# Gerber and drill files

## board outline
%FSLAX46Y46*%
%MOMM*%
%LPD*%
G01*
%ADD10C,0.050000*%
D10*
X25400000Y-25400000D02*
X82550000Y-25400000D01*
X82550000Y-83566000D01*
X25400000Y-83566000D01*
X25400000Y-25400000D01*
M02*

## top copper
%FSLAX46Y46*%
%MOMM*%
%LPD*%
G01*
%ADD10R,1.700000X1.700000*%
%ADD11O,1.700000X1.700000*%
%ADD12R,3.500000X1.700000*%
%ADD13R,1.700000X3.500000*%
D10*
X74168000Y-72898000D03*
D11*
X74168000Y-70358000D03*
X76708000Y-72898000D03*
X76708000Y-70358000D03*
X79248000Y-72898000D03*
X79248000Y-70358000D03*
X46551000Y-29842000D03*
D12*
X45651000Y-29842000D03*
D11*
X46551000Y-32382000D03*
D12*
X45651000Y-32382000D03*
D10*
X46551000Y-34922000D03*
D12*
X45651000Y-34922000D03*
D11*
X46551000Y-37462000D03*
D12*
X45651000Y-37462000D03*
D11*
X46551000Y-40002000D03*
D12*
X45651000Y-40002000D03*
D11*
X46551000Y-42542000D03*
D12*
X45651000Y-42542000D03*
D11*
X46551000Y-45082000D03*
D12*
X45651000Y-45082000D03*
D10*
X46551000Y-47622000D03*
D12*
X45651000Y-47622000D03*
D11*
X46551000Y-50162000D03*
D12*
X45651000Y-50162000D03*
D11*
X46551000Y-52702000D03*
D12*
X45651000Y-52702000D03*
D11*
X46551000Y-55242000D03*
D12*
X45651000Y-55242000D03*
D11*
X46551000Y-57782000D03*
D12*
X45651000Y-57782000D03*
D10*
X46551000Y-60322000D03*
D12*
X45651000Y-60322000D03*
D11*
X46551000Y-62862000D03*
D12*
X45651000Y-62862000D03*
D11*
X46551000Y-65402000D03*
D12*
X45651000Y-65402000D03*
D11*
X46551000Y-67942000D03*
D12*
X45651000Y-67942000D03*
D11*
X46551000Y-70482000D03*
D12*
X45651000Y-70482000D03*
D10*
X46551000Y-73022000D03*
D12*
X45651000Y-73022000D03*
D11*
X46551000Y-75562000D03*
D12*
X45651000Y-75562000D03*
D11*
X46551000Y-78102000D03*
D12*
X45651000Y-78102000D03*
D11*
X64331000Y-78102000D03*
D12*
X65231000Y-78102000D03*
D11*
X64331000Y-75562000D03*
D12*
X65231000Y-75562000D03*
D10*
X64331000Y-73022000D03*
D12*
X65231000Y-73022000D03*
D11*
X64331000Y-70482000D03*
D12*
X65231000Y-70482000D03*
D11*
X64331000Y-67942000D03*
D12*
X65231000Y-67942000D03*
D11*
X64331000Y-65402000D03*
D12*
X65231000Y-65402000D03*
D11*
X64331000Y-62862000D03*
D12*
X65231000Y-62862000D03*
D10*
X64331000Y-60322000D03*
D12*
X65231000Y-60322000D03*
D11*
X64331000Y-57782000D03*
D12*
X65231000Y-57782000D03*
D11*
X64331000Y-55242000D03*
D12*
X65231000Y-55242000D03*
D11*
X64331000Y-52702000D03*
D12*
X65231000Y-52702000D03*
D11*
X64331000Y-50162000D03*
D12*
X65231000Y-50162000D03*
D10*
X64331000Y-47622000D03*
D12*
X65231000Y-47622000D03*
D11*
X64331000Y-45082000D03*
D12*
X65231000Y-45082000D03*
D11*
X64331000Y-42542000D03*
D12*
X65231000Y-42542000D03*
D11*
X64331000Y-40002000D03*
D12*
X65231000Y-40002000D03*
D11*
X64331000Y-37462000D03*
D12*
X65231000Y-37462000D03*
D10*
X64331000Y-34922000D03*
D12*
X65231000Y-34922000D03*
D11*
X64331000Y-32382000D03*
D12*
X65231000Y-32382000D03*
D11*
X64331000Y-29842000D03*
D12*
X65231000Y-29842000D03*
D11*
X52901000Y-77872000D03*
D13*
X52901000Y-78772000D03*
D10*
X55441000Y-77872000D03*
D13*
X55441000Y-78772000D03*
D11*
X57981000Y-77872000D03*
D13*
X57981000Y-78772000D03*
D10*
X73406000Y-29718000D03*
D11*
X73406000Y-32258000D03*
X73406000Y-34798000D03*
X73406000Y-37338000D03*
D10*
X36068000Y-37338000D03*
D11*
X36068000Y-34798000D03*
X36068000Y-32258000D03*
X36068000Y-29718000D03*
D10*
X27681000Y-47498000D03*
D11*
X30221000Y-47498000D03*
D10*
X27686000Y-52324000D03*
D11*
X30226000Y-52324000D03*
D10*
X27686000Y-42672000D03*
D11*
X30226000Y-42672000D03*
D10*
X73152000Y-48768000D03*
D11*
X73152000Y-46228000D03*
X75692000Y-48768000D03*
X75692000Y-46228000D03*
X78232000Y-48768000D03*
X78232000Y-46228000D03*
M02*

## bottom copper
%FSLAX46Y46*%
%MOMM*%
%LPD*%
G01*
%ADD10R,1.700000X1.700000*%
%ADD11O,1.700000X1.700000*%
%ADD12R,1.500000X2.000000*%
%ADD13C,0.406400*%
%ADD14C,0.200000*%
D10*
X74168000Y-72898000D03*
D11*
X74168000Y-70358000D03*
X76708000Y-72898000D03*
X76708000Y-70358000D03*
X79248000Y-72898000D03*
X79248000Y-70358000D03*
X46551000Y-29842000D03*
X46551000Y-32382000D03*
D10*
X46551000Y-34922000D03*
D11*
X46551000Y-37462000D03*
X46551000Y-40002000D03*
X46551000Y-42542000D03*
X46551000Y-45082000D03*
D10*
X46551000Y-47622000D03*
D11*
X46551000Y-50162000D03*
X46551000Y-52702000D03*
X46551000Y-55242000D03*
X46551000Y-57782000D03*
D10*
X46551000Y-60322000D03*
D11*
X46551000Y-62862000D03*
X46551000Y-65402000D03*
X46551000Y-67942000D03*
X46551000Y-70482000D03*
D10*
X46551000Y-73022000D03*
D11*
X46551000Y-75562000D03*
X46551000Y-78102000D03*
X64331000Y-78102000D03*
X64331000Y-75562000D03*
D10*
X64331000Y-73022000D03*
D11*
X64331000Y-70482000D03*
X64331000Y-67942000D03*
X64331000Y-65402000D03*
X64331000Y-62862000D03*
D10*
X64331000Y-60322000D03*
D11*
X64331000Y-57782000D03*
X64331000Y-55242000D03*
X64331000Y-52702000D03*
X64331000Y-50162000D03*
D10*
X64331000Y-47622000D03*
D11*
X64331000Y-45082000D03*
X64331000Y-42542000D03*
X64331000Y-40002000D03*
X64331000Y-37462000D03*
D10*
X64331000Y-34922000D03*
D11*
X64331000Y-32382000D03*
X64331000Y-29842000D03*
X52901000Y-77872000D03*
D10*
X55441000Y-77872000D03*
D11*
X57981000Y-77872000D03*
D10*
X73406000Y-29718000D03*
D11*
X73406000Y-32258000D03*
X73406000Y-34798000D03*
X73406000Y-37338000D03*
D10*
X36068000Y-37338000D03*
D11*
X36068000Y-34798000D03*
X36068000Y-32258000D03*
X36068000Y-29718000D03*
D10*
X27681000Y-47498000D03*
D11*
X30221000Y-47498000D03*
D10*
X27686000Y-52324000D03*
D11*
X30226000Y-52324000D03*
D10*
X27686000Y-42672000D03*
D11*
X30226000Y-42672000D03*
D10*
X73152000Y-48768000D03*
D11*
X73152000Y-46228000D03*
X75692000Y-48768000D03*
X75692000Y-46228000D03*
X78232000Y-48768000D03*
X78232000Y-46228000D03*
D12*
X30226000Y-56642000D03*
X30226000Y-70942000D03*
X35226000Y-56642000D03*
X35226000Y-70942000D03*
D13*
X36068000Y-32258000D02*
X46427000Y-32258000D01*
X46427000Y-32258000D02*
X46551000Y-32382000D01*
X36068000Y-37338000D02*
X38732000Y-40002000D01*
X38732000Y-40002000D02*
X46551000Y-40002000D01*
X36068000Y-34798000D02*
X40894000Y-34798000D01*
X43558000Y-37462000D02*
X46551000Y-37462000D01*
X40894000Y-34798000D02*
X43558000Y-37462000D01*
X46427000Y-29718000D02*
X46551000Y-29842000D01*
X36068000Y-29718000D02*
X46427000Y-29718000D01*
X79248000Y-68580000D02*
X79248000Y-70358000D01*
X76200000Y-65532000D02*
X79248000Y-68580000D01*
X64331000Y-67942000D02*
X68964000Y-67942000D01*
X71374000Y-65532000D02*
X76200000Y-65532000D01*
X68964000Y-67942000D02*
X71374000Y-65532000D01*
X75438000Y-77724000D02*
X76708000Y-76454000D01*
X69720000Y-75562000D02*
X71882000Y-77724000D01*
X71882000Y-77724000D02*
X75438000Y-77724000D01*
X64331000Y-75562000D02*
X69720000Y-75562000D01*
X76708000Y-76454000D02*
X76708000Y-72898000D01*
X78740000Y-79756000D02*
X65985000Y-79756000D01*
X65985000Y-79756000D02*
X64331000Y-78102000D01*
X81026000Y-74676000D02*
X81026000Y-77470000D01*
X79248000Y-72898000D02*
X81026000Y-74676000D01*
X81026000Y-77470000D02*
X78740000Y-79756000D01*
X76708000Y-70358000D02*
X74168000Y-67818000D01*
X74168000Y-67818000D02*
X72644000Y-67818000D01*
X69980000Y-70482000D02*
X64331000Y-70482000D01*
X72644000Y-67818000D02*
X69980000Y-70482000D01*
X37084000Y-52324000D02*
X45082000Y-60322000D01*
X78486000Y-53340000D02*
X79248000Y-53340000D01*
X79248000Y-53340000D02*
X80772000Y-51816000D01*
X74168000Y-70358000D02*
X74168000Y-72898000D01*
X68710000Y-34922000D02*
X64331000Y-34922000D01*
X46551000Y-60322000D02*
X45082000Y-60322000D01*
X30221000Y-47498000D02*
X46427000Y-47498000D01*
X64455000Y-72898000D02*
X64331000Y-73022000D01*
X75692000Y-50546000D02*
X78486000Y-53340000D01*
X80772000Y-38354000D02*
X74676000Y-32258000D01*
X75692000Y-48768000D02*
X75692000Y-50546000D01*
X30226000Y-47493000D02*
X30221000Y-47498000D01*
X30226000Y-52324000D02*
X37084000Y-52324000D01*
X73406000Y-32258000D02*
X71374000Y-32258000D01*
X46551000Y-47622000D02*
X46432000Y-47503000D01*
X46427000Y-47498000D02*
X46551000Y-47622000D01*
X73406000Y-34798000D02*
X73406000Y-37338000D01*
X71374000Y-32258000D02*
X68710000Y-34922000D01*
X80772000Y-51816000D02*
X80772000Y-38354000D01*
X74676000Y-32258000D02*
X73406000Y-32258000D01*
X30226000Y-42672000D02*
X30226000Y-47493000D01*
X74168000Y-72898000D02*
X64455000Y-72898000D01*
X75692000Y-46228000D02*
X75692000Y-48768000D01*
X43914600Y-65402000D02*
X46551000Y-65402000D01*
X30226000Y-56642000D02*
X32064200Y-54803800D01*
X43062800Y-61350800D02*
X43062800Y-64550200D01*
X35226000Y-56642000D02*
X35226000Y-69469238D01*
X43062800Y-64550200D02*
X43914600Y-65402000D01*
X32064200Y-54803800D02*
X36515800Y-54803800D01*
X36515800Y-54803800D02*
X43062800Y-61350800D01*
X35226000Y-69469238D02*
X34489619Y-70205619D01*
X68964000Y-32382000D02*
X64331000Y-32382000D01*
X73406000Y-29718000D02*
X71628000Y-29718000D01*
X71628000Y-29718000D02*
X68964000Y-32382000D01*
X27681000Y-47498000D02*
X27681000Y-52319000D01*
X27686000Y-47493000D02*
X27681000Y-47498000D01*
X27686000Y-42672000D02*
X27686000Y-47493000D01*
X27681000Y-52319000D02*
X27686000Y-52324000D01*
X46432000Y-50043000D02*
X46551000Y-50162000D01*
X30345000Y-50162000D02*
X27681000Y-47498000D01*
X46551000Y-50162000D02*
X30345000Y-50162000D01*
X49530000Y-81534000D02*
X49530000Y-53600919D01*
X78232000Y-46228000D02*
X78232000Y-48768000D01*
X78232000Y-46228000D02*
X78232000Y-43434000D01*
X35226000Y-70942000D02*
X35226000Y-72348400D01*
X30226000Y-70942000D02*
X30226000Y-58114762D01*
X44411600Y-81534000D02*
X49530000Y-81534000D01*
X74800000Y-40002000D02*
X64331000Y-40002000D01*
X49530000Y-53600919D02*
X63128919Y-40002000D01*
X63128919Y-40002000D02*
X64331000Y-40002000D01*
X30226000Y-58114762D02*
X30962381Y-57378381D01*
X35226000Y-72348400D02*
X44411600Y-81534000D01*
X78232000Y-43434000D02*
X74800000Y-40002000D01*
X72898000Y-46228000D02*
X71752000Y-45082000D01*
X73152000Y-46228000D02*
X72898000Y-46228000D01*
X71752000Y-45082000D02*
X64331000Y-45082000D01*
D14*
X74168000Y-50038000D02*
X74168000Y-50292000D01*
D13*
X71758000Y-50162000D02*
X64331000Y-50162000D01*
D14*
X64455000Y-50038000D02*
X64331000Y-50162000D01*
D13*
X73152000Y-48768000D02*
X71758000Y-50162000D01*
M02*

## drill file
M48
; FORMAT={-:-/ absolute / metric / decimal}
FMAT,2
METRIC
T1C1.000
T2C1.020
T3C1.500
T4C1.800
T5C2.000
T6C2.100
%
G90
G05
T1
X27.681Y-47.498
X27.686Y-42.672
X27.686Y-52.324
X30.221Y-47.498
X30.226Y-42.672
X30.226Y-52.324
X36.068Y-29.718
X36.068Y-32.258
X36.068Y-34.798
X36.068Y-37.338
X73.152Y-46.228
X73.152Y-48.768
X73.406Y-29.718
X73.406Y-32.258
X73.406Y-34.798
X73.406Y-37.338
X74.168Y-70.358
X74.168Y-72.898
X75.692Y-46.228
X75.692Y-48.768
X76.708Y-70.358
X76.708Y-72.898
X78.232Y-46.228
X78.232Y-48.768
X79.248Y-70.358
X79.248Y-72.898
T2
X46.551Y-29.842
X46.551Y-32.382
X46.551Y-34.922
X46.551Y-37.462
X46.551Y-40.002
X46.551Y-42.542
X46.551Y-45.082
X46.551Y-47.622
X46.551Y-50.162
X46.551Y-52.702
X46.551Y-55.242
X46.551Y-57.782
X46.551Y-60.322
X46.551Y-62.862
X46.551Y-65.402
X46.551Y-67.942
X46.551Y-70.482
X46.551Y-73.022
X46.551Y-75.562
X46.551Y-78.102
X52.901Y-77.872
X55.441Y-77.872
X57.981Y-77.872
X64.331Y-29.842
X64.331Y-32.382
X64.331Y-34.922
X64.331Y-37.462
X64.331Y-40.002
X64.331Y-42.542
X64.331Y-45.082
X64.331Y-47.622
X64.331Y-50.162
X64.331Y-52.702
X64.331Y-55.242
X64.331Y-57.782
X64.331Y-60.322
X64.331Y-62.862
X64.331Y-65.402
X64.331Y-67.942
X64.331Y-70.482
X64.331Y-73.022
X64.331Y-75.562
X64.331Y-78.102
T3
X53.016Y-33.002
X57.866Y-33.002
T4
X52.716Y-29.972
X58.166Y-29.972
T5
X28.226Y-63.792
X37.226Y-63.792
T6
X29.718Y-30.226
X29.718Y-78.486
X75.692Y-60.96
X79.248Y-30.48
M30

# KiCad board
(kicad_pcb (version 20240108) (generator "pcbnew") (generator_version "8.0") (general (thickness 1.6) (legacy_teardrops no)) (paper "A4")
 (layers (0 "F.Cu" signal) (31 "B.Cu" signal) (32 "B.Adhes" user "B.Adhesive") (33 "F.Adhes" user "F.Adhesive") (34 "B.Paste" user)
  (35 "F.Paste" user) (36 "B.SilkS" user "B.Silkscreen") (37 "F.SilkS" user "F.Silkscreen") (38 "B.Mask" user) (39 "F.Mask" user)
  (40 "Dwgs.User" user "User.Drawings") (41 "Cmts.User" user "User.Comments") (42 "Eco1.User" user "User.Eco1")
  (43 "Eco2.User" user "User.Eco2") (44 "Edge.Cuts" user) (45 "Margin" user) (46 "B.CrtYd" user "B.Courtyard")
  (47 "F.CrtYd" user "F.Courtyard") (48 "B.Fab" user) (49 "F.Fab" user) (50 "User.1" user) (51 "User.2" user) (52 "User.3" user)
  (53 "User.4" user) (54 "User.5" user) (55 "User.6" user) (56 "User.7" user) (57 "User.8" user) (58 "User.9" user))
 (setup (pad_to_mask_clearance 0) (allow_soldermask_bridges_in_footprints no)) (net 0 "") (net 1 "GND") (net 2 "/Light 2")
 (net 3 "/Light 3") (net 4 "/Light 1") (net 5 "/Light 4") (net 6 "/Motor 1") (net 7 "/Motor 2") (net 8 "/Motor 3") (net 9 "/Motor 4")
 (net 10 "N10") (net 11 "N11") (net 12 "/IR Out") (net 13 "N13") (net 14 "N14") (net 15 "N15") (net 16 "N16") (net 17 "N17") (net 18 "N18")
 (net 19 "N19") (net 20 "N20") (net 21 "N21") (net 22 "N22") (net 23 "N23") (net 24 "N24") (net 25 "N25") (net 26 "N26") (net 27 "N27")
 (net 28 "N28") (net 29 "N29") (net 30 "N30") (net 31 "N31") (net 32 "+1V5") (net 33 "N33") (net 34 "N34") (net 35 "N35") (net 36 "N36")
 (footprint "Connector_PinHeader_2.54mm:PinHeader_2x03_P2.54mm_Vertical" (layer "F.Cu") (at 74.168 72.898 90)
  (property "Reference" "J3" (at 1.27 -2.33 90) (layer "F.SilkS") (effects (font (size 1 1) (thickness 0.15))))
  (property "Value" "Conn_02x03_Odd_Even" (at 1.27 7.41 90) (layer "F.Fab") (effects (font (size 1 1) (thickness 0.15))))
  (pad "1" thru_hole rect (at 0 0 90) (size 1.7 1.7) (drill 1) (layers "*.Cu" "*.Mask") (remove_unused_layers no) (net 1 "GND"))
  (pad "2" thru_hole oval (at 2.54 0 90) (size 1.7 1.7) (drill 1) (layers "*.Cu" "*.Mask") (remove_unused_layers no) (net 1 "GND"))
  (pad "3" thru_hole oval (at 0 2.54 90) (size 1.7 1.7) (drill 1) (layers "*.Cu" "*.Mask") (remove_unused_layers no) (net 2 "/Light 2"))
  (pad "4" thru_hole oval (at 2.54 2.54 90) (size 1.7 1.7) (drill 1) (layers "*.Cu" "*.Mask") (remove_unused_layers no) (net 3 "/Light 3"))
  (pad "5" thru_hole oval (at 0 5.08 90) (size 1.7 1.7) (drill 1) (layers "*.Cu" "*.Mask") (remove_unused_layers no) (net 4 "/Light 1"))
  (pad "6" thru_hole oval (at 2.54 5.08 90) (size 1.7 1.7) (drill 1) (layers "*.Cu" "*.Mask") (remove_unused_layers no) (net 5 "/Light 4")))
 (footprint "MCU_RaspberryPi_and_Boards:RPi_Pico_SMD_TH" (layer "F.Cu") (at 55.441 53.972)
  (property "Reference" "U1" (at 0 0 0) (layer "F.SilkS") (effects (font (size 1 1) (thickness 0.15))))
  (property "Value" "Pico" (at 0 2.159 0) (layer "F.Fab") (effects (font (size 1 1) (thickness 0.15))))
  (pad "" np_thru_hole oval (at -2.725 -24) (size 1.8 1.8) (drill 1.8) (layers "*.Cu" "*.Mask"))
  (pad "" np_thru_hole oval (at -2.425 -20.97) (size 1.5 1.5) (drill 1.5) (layers "*.Cu" "*.Mask"))
  (pad "" np_thru_hole oval (at 2.425 -20.97) (size 1.5 1.5) (drill 1.5) (layers "*.Cu" "*.Mask"))
  (pad "" np_thru_hole oval (at 2.725 -24) (size 1.8 1.8) (drill 1.8) (layers "*.Cu" "*.Mask"))
  (pad "1" thru_hole oval (at -8.89 -24.13) (size 1.7 1.7) (drill 1.02) (layers "*.Cu" "*.Mask") (remove_unused_layers no)
   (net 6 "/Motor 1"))
  (pad "1" smd rect (at -8.89 -24.13) (size 3.5 1.7) (drill (offset -0.9 0)) (layers "F.Cu" "F.Mask") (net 6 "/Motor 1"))
  (pad "2" thru_hole oval (at -8.89 -21.59) (size 1.7 1.7) (drill 1.02) (layers "*.Cu" "*.Mask") (remove_unused_layers no)
   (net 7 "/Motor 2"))
  (pad "2" smd rect (at -8.89 -21.59) (size 3.5 1.7) (drill (offset -0.9 0)) (layers "F.Cu" "F.Mask") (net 7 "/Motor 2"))
  (pad "3" thru_hole rect (at -8.89 -19.05) (size 1.7 1.7) (drill 1.02) (layers "*.Cu" "*.Mask") (remove_unused_layers no) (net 1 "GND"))
  (pad "3" smd rect (at -8.89 -19.05) (size 3.5 1.7) (drill (offset -0.9 0)) (layers "F.Cu" "F.Mask") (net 1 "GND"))
  (pad "4" thru_hole oval (at -8.89 -16.51) (size 1.7 1.7) (drill 1.02) (layers "*.Cu" "*.Mask") (remove_unused_layers no)
   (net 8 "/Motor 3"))
  (pad "4" smd rect (at -8.89 -16.51) (size 3.5 1.7) (drill (offset -0.9 0)) (layers "F.Cu" "F.Mask") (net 8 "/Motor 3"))
  (pad "5" thru_hole oval (at -8.89 -13.97) (size 1.7 1.7) (drill 1.02) (layers "*.Cu" "*.Mask") (remove_unused_layers no)
   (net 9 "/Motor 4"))
  (pad "5" smd rect (at -8.89 -13.97) (size 3.5 1.7) (drill (offset -0.9 0)) (layers "F.Cu" "F.Mask") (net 9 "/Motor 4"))
  (pad "6" thru_hole oval (at -8.89 -11.43) (size 1.7 1.7) (drill 1.02) (layers "*.Cu" "*.Mask") (remove_unused_layers no) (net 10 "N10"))
  (pad "6" smd rect (at -8.89 -11.43) (size 3.5 1.7) (drill (offset -0.9 0)) (layers "F.Cu" "F.Mask") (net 10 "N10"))
  (pad "7" thru_hole oval (at -8.89 -8.89) (size 1.7 1.7) (drill 1.02) (layers "*.Cu" "*.Mask") (remove_unused_layers no) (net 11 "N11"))
  (pad "7" smd rect (at -8.89 -8.89) (size 3.5 1.7) (drill (offset -0.9 0)) (layers "F.Cu" "F.Mask") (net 11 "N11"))
  (pad "8" thru_hole rect (at -8.89 -6.35) (size 1.7 1.7) (drill 1.02) (layers "*.Cu" "*.Mask") (remove_unused_layers no) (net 1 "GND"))
  (pad "8" smd rect (at -8.89 -6.35) (size 3.5 1.7) (drill (offset -0.9 0)) (layers "F.Cu" "F.Mask") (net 1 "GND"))
  (pad "9" thru_hole oval (at -8.89 -3.81) (size 1.7 1.7) (drill 1.02) (layers "*.Cu" "*.Mask") (remove_unused_layers no) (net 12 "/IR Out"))
  (pad "9" smd rect (at -8.89 -3.81) (size 3.5 1.7) (drill (offset -0.9 0)) (layers "F.Cu" "F.Mask") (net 12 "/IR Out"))
  (pad "10" thru_hole oval (at -8.89 -1.27) (size 1.7 1.7) (drill 1.02) (layers "*.Cu" "*.Mask") (remove_unused_layers no) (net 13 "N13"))
  (pad "10" smd rect (at -8.89 -1.27) (size 3.5 1.7) (drill (offset -0.9 0)) (layers "F.Cu" "F.Mask") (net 13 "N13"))
  (pad "11" thru_hole oval (at -8.89 1.27) (size 1.7 1.7) (drill 1.02) (layers "*.Cu" "*.Mask") (remove_unused_layers no) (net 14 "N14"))
  (pad "11" smd rect (at -8.89 1.27) (size 3.5 1.7) (drill (offset -0.9 0)) (layers "F.Cu" "F.Mask") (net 14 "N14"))
  (pad "12" thru_hole oval (at -8.89 3.81) (size 1.7 1.7) (drill 1.02) (layers "*.Cu" "*.Mask") (remove_unused_layers no) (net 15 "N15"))
  (pad "12" smd rect (at -8.89 3.81) (size 3.5 1.7) (drill (offset -0.9 0)) (layers "F.Cu" "F.Mask") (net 15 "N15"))
  (pad "13" thru_hole rect (at -8.89 6.35) (size 1.7 1.7) (drill 1.02) (layers "*.Cu" "*.Mask") (remove_unused_layers no) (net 1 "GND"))
  (pad "13" smd rect (at -8.89 6.35) (size 3.5 1.7) (drill (offset -0.9 0)) (layers "F.Cu" "F.Mask") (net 1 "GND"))
  (pad "14" thru_hole oval (at -8.89 8.89) (size 1.7 1.7) (drill 1.02) (layers "*.Cu" "*.Mask") (remove_unused_layers no) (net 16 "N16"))
  (pad "14" smd rect (at -8.89 8.89) (size 3.5 1.7) (drill (offset -0.9 0)) (layers "F.Cu" "F.Mask") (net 16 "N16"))
  (pad "15" thru_hole oval (at -8.89 11.43) (size 1.7 1.7) (drill 1.02) (layers "*.Cu" "*.Mask") (remove_unused_layers no) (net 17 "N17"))
  (pad "15" smd rect (at -8.89 11.43) (size 3.5 1.7) (drill (offset -0.9 0)) (layers "F.Cu" "F.Mask") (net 17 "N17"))
  (pad "16" thru_hole oval (at -8.89 13.97) (size 1.7 1.7) (drill 1.02) (layers "*.Cu" "*.Mask") (remove_unused_layers no) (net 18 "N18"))
  (pad "16" smd rect (at -8.89 13.97) (size 3.5 1.7) (drill (offset -0.9 0)) (layers "F.Cu" "F.Mask") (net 18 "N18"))
  (pad "17" thru_hole oval (at -8.89 16.51) (size 1.7 1.7) (drill 1.02) (layers "*.Cu" "*.Mask") (remove_unused_layers no) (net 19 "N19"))
  (pad "17" smd rect (at -8.89 16.51) (size 3.5 1.7) (drill (offset -0.9 0)) (layers "F.Cu" "F.Mask") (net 19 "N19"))
  (pad "18" thru_hole rect (at -8.89 19.05) (size 1.7 1.7) (drill 1.02) (layers "*.Cu" "*.Mask") (remove_unused_layers no) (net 1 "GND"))
  (pad "18" smd rect (at -8.89 19.05) (size 3.5 1.7) (drill (offset -0.9 0)) (layers "F.Cu" "F.Mask") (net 1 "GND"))
  (pad "19" thru_hole oval (at -8.89 21.59) (size 1.7 1.7) (drill 1.02) (layers "*.Cu" "*.Mask") (remove_unused_layers no) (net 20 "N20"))
  (pad "19" smd rect (at -8.89 21.59) (size 3.5 1.7) (drill (offset -0.9 0)) (layers "F.Cu" "F.Mask") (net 20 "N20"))
  (pad "20" thru_hole oval (at -8.89 24.13) (size 1.7 1.7) (drill 1.02) (layers "*.Cu" "*.Mask") (remove_unused_layers no) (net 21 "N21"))
  (pad "20" smd rect (at -8.89 24.13) (size 3.5 1.7) (drill (offset -0.9 0)) (layers "F.Cu" "F.Mask") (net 21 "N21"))
  (pad "21" thru_hole oval (at 8.89 24.13) (size 1.7 1.7) (drill 1.02) (layers "*.Cu" "*.Mask") (remove_unused_layers no) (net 4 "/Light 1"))
  (pad "21" smd rect (at 8.89 24.13) (size 3.5 1.7) (drill (offset 0.9 0)) (layers "F.Cu" "F.Mask") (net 4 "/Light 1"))
  (pad "22" thru_hole oval (at 8.89 21.59) (size 1.7 1.7) (drill 1.02) (layers "*.Cu" "*.Mask") (remove_unused_layers no) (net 2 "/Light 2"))
  (pad "22" smd rect (at 8.89 21.59) (size 3.5 1.7) (drill (offset 0.9 0)) (layers "F.Cu" "F.Mask") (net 2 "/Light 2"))
  (pad "23" thru_hole rect (at 8.89 19.05) (size 1.7 1.7) (drill 1.02) (layers "*.Cu" "*.Mask") (remove_unused_layers no) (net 1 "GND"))
  (pad "23" smd rect (at 8.89 19.05) (size 3.5 1.7) (drill (offset 0.9 0)) (layers "F.Cu" "F.Mask") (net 1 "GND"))
  (pad "24" thru_hole oval (at 8.89 16.51) (size 1.7 1.7) (drill 1.02) (layers "*.Cu" "*.Mask") (remove_unused_layers no) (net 3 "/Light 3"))
  (pad "24" smd rect (at 8.89 16.51) (size 3.5 1.7) (drill (offset 0.9 0)) (layers "F.Cu" "F.Mask") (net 3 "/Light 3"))
  (pad "25" thru_hole oval (at 8.89 13.97) (size 1.7 1.7) (drill 1.02) (layers "*.Cu" "*.Mask") (remove_unused_layers no) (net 5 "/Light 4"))
  (pad "25" smd rect (at 8.89 13.97) (size 3.5 1.7) (drill (offset 0.9 0)) (layers "F.Cu" "F.Mask") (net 5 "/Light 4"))
  (pad "26" thru_hole oval (at 8.89 11.43) (size 1.7 1.7) (drill 1.02) (layers "*.Cu" "*.Mask") (remove_unused_layers no) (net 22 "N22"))
  (pad "26" smd rect (at 8.89 11.43) (size 3.5 1.7) (drill (offset 0.9 0)) (layers "F.Cu" "F.Mask") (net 22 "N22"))
  (pad "27" thru_hole oval (at 8.89 8.89) (size 1.7 1.7) (drill 1.02) (layers "*.Cu" "*.Mask") (remove_unused_layers no) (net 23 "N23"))
  (pad "27" smd rect (at 8.89 8.89) (size 3.5 1.7) (drill (offset 0.9 0)) (layers "F.Cu" "F.Mask") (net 23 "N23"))
  (pad "28" thru_hole rect (at 8.89 6.35) (size 1.7 1.7) (drill 1.02) (layers "*.Cu" "*.Mask") (remove_unused_layers no) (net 1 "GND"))
  (pad "28" smd rect (at 8.89 6.35) (size 3.5 1.7) (drill (offset 0.9 0)) (layers "F.Cu" "F.Mask") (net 1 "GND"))
  (pad "29" thru_hole oval (at 8.89 3.81) (size 1.7 1.7) (drill 1.02) (layers "*.Cu" "*.Mask") (remove_unused_layers no) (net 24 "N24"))
  (pad "29" smd rect (at 8.89 3.81) (size 3.5 1.7) (drill (offset 0.9 0)) (layers "F.Cu" "F.Mask") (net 24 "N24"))
  (pad "30" thru_hole oval (at 8.89 1.27) (size 1.7 1.7) (drill 1.02) (layers "*.Cu" "*.Mask") (remove_unused_layers no) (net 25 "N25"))
  (pad "30" smd rect (at 8.89 1.27) (size 3.5 1.7) (drill (offset 0.9 0)) (layers "F.Cu" "F.Mask") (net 25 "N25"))
  (pad "31" thru_hole oval (at 8.89 -1.27) (size 1.7 1.7) (drill 1.02) (layers "*.Cu" "*.Mask") (remove_unused_layers no) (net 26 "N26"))
  (pad "31" smd rect (at 8.89 -1.27) (size 3.5 1.7) (drill (offset 0.9 0)) (layers "F.Cu" "F.Mask") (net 26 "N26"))
  (pad "32" thru_hole oval (at 8.89 -3.81) (size 1.7 1.7) (drill 1.02) (layers "*.Cu" "*.Mask") (remove_unused_layers no) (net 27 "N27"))
  (pad "32" smd rect (at 8.89 -3.81) (size 3.5 1.7) (drill (offset 0.9 0)) (layers "F.Cu" "F.Mask") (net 27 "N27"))
  (pad "33" thru_hole rect (at 8.89 -6.35) (size 1.7 1.7) (drill 1.02) (layers "*.Cu" "*.Mask") (remove_unused_layers no) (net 1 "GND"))
  (pad "33" smd rect (at 8.89 -6.35) (size 3.5 1.7) (drill (offset 0.9 0)) (layers "F.Cu" "F.Mask") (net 1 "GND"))
  (pad "34" thru_hole oval (at 8.89 -8.89) (size 1.7 1.7) (drill 1.02) (layers "*.Cu" "*.Mask") (remove_unused_layers no) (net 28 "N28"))
  (pad "34" smd rect (at 8.89 -8.89) (size 3.5 1.7) (drill (offset 0.9 0)) (layers "F.Cu" "F.Mask") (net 28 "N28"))
  (pad "35" thru_hole oval (at 8.89 -11.43) (size 1.7 1.7) (drill 1.02) (layers "*.Cu" "*.Mask") (remove_unused_layers no) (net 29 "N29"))
  (pad "35" smd rect (at 8.89 -11.43) (size 3.5 1.7) (drill (offset 0.9 0)) (layers "F.Cu" "F.Mask") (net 29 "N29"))
  (pad "36" thru_hole oval (at 8.89 -13.97) (size 1.7 1.7) (drill 1.02) (layers "*.Cu" "*.Mask") (remove_unused_layers no) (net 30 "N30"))
  (pad "36" smd rect (at 8.89 -13.97) (size 3.5 1.7) (drill (offset 0.9 0)) (layers "F.Cu" "F.Mask") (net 30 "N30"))
  (pad "37" thru_hole oval (at 8.89 -16.51) (size 1.7 1.7) (drill 1.02) (layers "*.Cu" "*.Mask") (remove_unused_layers no) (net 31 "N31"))
  (pad "37" smd rect (at 8.89 -16.51) (size 3.5 1.7) (drill (offset 0.9 0)) (layers "F.Cu" "F.Mask") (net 31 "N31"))
  (pad "38" thru_hole rect (at 8.89 -19.05) (size 1.7 1.7) (drill 1.02) (layers "*.Cu" "*.Mask") (remove_unused_layers no) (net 1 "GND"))
  (pad "38" smd rect (at 8.89 -19.05) (size 3.5 1.7) (drill (offset 0.9 0)) (layers "F.Cu" "F.Mask") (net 1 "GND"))
  (pad "39" thru_hole oval (at 8.89 -21.59) (size 1.7 1.7) (drill 1.02) (layers "*.Cu" "*.Mask") (remove_unused_layers no) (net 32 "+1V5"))
  (pad "39" smd rect (at 8.89 -21.59) (size 3.5 1.7) (drill (offset 0.9 0)) (layers "F.Cu" "F.Mask") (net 32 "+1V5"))
  (pad "40" thru_hole oval (at 8.89 -24.13) (size 1.7 1.7) (drill 1.02) (layers "*.Cu" "*.Mask") (remove_unused_layers no) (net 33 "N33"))
  (pad "40" smd rect (at 8.89 -24.13) (size 3.5 1.7) (drill (offset 0.9 0)) (layers "F.Cu" "F.Mask") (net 33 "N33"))
  (pad "41" thru_hole oval (at -2.54 23.9) (size 1.7 1.7) (drill 1.02) (layers "*.Cu" "*.Mask") (remove_unused_layers no) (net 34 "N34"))
  (pad "41" smd rect (at -2.54 23.9 90) (size 3.5 1.7) (drill (offset -0.9 0)) (layers "F.Cu" "F.Mask") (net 34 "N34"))
  (pad "42" thru_hole rect (at 0 23.9) (size 1.7 1.7) (drill 1.02) (layers "*.Cu" "*.Mask") (remove_unused_layers no) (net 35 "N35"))
  (pad "42" smd rect (at 0 23.9 90) (size 3.5 1.7) (drill (offset -0.9 0)) (layers "F.Cu" "F.Mask") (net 35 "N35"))
  (pad "43" thru_hole oval (at 2.54 23.9) (size 1.7 1.7) (drill 1.02) (layers "*.Cu" "*.Mask") (remove_unused_layers no) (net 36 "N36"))
  (pad "43" smd rect (at 2.54 23.9 90) (size 3.5 1.7) (drill (offset -0.9 0)) (layers "F.Cu" "F.Mask") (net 36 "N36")))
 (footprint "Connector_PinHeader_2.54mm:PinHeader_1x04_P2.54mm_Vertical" (layer "F.Cu") (at 73.406 29.718)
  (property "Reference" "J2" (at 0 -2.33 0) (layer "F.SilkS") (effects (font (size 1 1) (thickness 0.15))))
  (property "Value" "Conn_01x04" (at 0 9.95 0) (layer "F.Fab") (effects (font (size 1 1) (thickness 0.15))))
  (pad "1" thru_hole rect (at 0 0) (size 1.7 1.7) (drill 1) (layers "*.Cu" "*.Mask") (remove_unused_layers no) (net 32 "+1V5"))
  (pad "2" thru_hole oval (at 0 2.54) (size 1.7 1.7) (drill 1) (layers "*.Cu" "*.Mask") (remove_unused_layers no) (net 1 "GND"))
  (pad "3" thru_hole oval (at 0 5.08) (size 1.7 1.7) (drill 1) (layers "*.Cu" "*.Mask") (remove_unused_layers no) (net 1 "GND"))
  (pad "4" thru_hole oval (at 0 7.62) (size 1.7 1.7) (drill 1) (layers "*.Cu" "*.Mask") (remove_unused_layers no) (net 1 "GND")))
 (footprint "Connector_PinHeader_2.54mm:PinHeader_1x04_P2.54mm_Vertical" (layer "F.Cu") (at 36.068 37.338 180)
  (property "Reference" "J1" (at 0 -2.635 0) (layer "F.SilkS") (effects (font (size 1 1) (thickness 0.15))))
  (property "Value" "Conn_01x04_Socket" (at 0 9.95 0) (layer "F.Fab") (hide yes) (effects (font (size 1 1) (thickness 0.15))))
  (pad "1" thru_hole rect (at 0 0 180) (size 1.7 1.7) (drill 1) (layers "*.Cu" "*.Mask") (remove_unused_layers no) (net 9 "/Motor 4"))
  (pad "2" thru_hole oval (at 0 2.54 180) (size 1.7 1.7) (drill 1) (layers "*.Cu" "*.Mask") (remove_unused_layers no) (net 8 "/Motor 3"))
  (pad "3" thru_hole oval (at 0 5.08 180) (size 1.7 1.7) (drill 1) (layers "*.Cu" "*.Mask") (remove_unused_layers no) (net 7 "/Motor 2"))
  (pad "4" thru_hole oval (at 0 7.62 180) (size 1.7 1.7) (drill 1) (layers "*.Cu" "*.Mask") (remove_unused_layers no) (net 6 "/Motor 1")))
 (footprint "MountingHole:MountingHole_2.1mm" (layer "F.Cu") (at 29.718 78.486)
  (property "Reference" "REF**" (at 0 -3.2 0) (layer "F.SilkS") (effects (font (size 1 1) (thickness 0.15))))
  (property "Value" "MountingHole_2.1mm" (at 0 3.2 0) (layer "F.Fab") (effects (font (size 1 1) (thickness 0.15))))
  (pad "" np_thru_hole circle (at 0 0) (size 2.1 2.1) (drill 2.1) (layers "*.Cu" "*.Mask")))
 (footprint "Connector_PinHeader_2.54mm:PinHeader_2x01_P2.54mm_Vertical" (layer "F.Cu") (at 27.681 47.498)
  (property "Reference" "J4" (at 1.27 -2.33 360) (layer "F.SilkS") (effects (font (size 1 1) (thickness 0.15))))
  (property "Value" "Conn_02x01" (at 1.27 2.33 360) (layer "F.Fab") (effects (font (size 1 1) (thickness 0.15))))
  (pad "1" thru_hole rect (at 0 0) (size 1.7 1.7) (drill 1) (layers "*.Cu" "*.Mask") (remove_unused_layers no) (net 12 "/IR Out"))
  (pad "2" thru_hole oval (at 2.54 0) (size 1.7 1.7) (drill 1) (layers "*.Cu" "*.Mask") (remove_unused_layers no) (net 1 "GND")))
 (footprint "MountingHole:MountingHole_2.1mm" (layer "F.Cu") (at 75.692 60.96)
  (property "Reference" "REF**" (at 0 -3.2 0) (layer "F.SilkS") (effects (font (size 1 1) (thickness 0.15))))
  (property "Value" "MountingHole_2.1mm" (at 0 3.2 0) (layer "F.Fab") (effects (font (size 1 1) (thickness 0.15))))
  (pad "" np_thru_hole circle (at 0 0) (size 2.1 2.1) (drill 2.1) (layers "F&B.Cu" "*.Mask")))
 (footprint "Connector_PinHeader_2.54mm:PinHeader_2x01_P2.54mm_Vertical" (layer "F.Cu") (at 27.686 52.324)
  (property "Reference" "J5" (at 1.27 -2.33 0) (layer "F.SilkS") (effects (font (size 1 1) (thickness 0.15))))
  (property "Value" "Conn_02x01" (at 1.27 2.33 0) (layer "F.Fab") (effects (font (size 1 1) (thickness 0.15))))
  (pad "1" thru_hole rect (at 0 0) (size 1.7 1.7) (drill 1) (layers "*.Cu" "*.Mask") (remove_unused_layers no) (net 12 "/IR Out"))
  (pad "2" thru_hole oval (at 2.54 0) (size 1.7 1.7) (drill 1) (layers "*.Cu" "*.Mask") (remove_unused_layers no) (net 1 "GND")))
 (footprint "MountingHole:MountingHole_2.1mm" (layer "F.Cu") (at 79.248 30.48)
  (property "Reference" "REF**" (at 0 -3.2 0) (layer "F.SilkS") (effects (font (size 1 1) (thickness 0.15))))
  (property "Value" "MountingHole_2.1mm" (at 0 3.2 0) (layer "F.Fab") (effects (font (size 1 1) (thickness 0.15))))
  (pad "" np_thru_hole circle (at 0 0) (size 2.1 2.1) (drill 2.1) (layers "F&B.Cu" "*.Mask")))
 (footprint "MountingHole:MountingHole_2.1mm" (layer "F.Cu") (at 29.718 30.226)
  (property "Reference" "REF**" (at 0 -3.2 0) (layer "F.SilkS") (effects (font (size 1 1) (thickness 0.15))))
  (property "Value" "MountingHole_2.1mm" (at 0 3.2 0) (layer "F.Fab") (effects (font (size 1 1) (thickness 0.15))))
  (pad "" np_thru_hole circle (at 0 0) (size 2.1 2.1) (drill 2.1) (layers "F&B.Cu" "*.Mask")))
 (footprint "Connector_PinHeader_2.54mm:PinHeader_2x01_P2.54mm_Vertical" (layer "F.Cu") (at 27.686 42.672)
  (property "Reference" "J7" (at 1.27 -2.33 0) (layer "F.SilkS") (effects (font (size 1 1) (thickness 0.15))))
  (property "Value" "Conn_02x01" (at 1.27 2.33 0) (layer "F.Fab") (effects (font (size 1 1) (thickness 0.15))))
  (pad "1" thru_hole rect (at 0 0) (size 1.7 1.7) (drill 1) (layers "*.Cu" "*.Mask") (remove_unused_layers no) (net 12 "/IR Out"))
  (pad "2" thru_hole oval (at 2.54 0) (size 1.7 1.7) (drill 1) (layers "*.Cu" "*.Mask") (remove_unused_layers no) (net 1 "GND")))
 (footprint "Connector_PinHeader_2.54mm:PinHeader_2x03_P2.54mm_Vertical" (layer "F.Cu") (at 73.152 48.768 90)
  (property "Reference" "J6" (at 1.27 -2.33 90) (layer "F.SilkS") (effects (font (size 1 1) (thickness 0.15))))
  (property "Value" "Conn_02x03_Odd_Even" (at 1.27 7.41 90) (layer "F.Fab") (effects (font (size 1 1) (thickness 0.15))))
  (pad "1" thru_hole rect (at 0 0 90) (size 1.7 1.7) (drill 1) (layers "*.Cu" "*.Mask") (remove_unused_layers no) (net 27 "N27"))
  (pad "2" thru_hole oval (at 2.54 0 90) (size 1.7 1.7) (drill 1) (layers "*.Cu" "*.Mask") (remove_unused_layers no) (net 28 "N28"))
  (pad "3" thru_hole oval (at 0 2.54 90) (size 1.7 1.7) (drill 1) (layers "*.Cu" "*.Mask") (remove_unused_layers no) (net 1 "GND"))
  (pad "4" thru_hole oval (at 2.54 2.54 90) (size 1.7 1.7) (drill 1) (layers "*.Cu" "*.Mask") (remove_unused_layers no) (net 1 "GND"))
  (pad "5" thru_hole oval (at 0 5.08 90) (size 1.7 1.7) (drill 1) (layers "*.Cu" "*.Mask") (remove_unused_layers no) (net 30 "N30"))
  (pad "6" thru_hole oval (at 2.54 5.08 90) (size 1.7 1.7) (drill 1) (layers "*.Cu" "*.Mask") (remove_unused_layers no) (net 30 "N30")))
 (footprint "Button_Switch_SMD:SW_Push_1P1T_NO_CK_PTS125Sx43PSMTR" (layer "B.Cu") (at 32.726 63.792 -90)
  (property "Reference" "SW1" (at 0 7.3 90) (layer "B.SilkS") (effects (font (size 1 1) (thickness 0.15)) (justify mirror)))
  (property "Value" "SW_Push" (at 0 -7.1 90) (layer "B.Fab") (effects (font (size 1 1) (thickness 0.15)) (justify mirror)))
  (pad "" np_thru_hole circle (at 0 -4.5 270) (size 2 2) (drill 2) (layers "*.Cu" "*.Mask"))
  (pad "" np_thru_hole circle (at 0 4.5 270) (size 2 2) (drill 2) (layers "*.Cu" "*.Mask"))
  (pad "1" smd rect (at -7.15 2.5 270) (size 2 1.5) (layers "B.Cu" "B.Paste" "B.Mask") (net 30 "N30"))
  (pad "1" smd rect (at 7.15 2.5 270) (size 2 1.5) (layers "B.Cu" "B.Paste" "B.Mask") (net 30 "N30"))
  (pad "2" smd rect (at -7.15 -2.5 270) (size 2 1.5) (layers "B.Cu" "B.Paste" "B.Mask") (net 17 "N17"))
  (pad "2" smd rect (at 7.15 -2.5 270) (size 2 1.5) (layers "B.Cu" "B.Paste" "B.Mask") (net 17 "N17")))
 (gr_rect (start 25.4 25.4) (end 82.55 83.566) (stroke (width 0.05) (type default)) (fill none) (layer "Edge.Cuts"))
 (segment (start 36.068 32.258) (end 46.427 32.258) (width 0.4064) (layer "B.Cu") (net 7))
 (segment (start 46.427 32.258) (end 46.551 32.382) (width 0.4064) (layer "B.Cu") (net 7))
 (segment (start 36.068 37.338) (end 38.732 40.002) (width 0.4064) (layer "B.Cu") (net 9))
 (segment (start 38.732 40.002) (end 46.551 40.002) (width 0.4064) (layer "B.Cu") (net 9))
 (segment (start 36.068 34.798) (end 40.894 34.798) (width 0.4064) (layer "B.Cu") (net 8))
 (segment (start 43.558 37.462) (end 46.551 37.462) (width 0.4064) (layer "B.Cu") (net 8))
 (segment (start 40.894 34.798) (end 43.558 37.462) (width 0.4064) (layer "B.Cu") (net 8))
 (segment (start 46.427 29.718) (end 46.551 29.842) (width 0.4064) (layer "B.Cu") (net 6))
 (segment (start 36.068 29.718) (end 46.427 29.718) (width 0.4064) (layer "B.Cu") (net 6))
 (segment (start 79.248 68.58) (end 79.248 70.358) (width 0.4064) (layer "B.Cu") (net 5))
 (segment (start 76.2 65.532) (end 79.248 68.58) (width 0.4064) (layer "B.Cu") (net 5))
 (segment (start 64.331 67.942) (end 68.964 67.942) (width 0.4064) (layer "B.Cu") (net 5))
 (segment (start 71.374 65.532) (end 76.2 65.532) (width 0.4064) (layer "B.Cu") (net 5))
 (segment (start 68.964 67.942) (end 71.374 65.532) (width 0.4064) (layer "B.Cu") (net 5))
 (segment (start 75.438 77.724) (end 76.708 76.454) (width 0.4064) (layer "B.Cu") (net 2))
 (segment (start 69.72 75.562) (end 71.882 77.724) (width 0.4064) (layer "B.Cu") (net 2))
 (segment (start 71.882 77.724) (end 75.438 77.724) (width 0.4064) (layer "B.Cu") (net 2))
 (segment (start 64.331 75.562) (end 69.72 75.562) (width 0.4064) (layer "B.Cu") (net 2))
 (segment (start 76.708 76.454) (end 76.708 72.898) (width 0.4064) (layer "B.Cu") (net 2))
 (segment (start 78.74 79.756) (end 65.985 79.756) (width 0.4064) (layer "B.Cu") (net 4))
 (segment (start 65.985 79.756) (end 64.331 78.102) (width 0.4064) (layer "B.Cu") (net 4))
 (segment (start 81.026 74.676) (end 81.026 77.47) (width 0.4064) (layer "B.Cu") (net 4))
 (segment (start 79.248 72.898) (end 81.026 74.676) (width 0.4064) (layer "B.Cu") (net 4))
 (segment (start 81.026 77.47) (end 78.74 79.756) (width 0.4064) (layer "B.Cu") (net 4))
 (segment (start 76.708 70.358) (end 74.168 67.818) (width 0.4064) (layer "B.Cu") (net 3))
 (segment (start 74.168 67.818) (end 72.644 67.818) (width 0.4064) (layer "B.Cu") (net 3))
 (segment (start 69.98 70.482) (end 64.331 70.482) (width 0.4064) (layer "B.Cu") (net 3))
 (segment (start 72.644 67.818) (end 69.98 70.482) (width 0.4064) (layer "B.Cu") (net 3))
 (segment (start 37.084 52.324) (end 45.082 60.322) (width 0.4064) (layer "B.Cu") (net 1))
 (segment (start 78.486 53.34) (end 79.248 53.34) (width 0.4064) (layer "B.Cu") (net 1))
 (segment (start 79.248 53.34) (end 80.772 51.816) (width 0.4064) (layer "B.Cu") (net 1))
 (segment (start 74.168 70.358) (end 74.168 72.898) (width 0.4064) (layer "B.Cu") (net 1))
 (segment (start 68.71 34.922) (end 64.331 34.922) (width 0.4064) (layer "B.Cu") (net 1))
 (segment (start 46.551 60.322) (end 45.082 60.322) (width 0.4064) (layer "B.Cu") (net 1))
 (segment (start 30.221 47.498) (end 46.427 47.498) (width 0.4064) (layer "B.Cu") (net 1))
 (segment (start 64.455 72.898) (end 64.331 73.022) (width 0.4064) (layer "B.Cu") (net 1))
 (segment (start 75.692 50.546) (end 78.486 53.34) (width 0.4064) (layer "B.Cu") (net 1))
 (segment (start 80.772 38.354) (end 74.676 32.258) (width 0.4064) (layer "B.Cu") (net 1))
 (segment (start 75.692 48.768) (end 75.692 50.546) (width 0.4064) (layer "B.Cu") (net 1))
 (segment (start 30.226 47.493) (end 30.221 47.498) (width 0.4064) (layer "B.Cu") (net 1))
 (segment (start 30.226 52.324) (end 37.084 52.324) (width 0.4064) (layer "B.Cu") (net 1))
 (segment (start 73.406 32.258) (end 71.374 32.258) (width 0.4064) (layer "B.Cu") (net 1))
 (segment (start 46.551 47.622) (end 46.432 47.503) (width 0.4064) (layer "B.Cu") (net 1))
 (segment (start 46.427 47.498) (end 46.551 47.622) (width 0.4064) (layer "B.Cu") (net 1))
 (segment (start 73.406 34.798) (end 73.406 37.338) (width 0.4064) (layer "B.Cu") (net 1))
 (segment (start 71.374 32.258) (end 68.71 34.922) (width 0.4064) (layer "B.Cu") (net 1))
 (segment (start 80.772 51.816) (end 80.772 38.354) (width 0.4064) (layer "B.Cu") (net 1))
 (segment (start 74.676 32.258) (end 73.406 32.258) (width 0.4064) (layer "B.Cu") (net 1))
 (segment (start 30.226 42.672) (end 30.226 47.493) (width 0.4064) (layer "B.Cu") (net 1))
 (segment (start 74.168 72.898) (end 64.455 72.898) (width 0.4064) (layer "B.Cu") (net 1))
 (segment (start 75.692 46.228) (end 75.692 48.768) (width 0.4064) (layer "B.Cu") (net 1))
 (segment (start 43.9146 65.402) (end 46.551 65.402) (width 0.4064) (layer "B.Cu") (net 17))
 (segment (start 30.226 56.642) (end 32.0642 54.8038) (width 0.4064) (layer "B.Cu") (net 17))
 (segment (start 43.0628 61.3508) (end 43.0628 64.5502) (width 0.4064) (layer "B.Cu") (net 17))
 (segment (start 35.226 56.642) (end 35.226 69.469238) (width 0.4064) (layer "B.Cu") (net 17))
 (segment (start 43.0628 64.5502) (end 43.9146 65.402) (width 0.4064) (layer "B.Cu") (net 17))
 (segment (start 32.0642 54.8038) (end 36.5158 54.8038) (width 0.4064) (layer "B.Cu") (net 17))
 (segment (start 36.5158 54.8038) (end 43.0628 61.3508) (width 0.4064) (layer "B.Cu") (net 17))
 (segment (start 35.226 69.469238) (end 34.489619 70.205619) (width 0.4064) (layer "B.Cu") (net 17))
 (segment (start 68.964 32.382) (end 64.331 32.382) (width 0.4064) (layer "B.Cu") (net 32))
 (segment (start 73.406 29.718) (end 71.628 29.718) (width 0.4064) (layer "B.Cu") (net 32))
 (segment (start 71.628 29.718) (end 68.964 32.382) (width 0.4064) (layer "B.Cu") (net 32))
 (segment (start 27.681 47.498) (end 27.681 52.319) (width 0.4064) (layer "B.Cu") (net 12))
 (segment (start 27.686 47.493) (end 27.681 47.498) (width 0.4064) (layer "B.Cu") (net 12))
 (segment (start 27.686 42.672) (end 27.686 47.493) (width 0.4064) (layer "B.Cu") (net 12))
 (segment (start 27.681 52.319) (end 27.686 52.324) (width 0.4064) (layer "B.Cu") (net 12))
 (segment (start 46.432 50.043) (end 46.551 50.162) (width 0.4064) (layer "B.Cu") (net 12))
 (segment (start 30.345 50.162) (end 27.681 47.498) (width 0.4064) (layer "B.Cu") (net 12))
 (segment (start 46.551 50.162) (end 30.345 50.162) (width 0.4064) (layer "B.Cu") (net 12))
 (segment (start 49.53 81.534) (end 49.53 53.600919) (width 0.4064) (layer "B.Cu") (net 30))
 (segment (start 78.232 46.228) (end 78.232 48.768) (width 0.4064) (layer "B.Cu") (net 30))
 (segment (start 78.232 46.228) (end 78.232 43.434) (width 0.4064) (layer "B.Cu") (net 30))
 (segment (start 35.226 70.942) (end 35.226 72.3484) (width 0.4064) (layer "B.Cu") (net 30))
 (segment (start 30.226 70.942) (end 30.226 58.114762) (width 0.4064) (layer "B.Cu") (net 30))
 (segment (start 44.4116 81.534) (end 49.53 81.534) (width 0.4064) (layer "B.Cu") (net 30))
 (segment (start 74.8 40.002) (end 64.331 40.002) (width 0.4064) (layer "B.Cu") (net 30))
 (segment (start 49.53 53.600919) (end 63.128919 40.002) (width 0.4064) (layer "B.Cu") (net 30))
 (segment (start 63.128919 40.002) (end 64.331 40.002) (width 0.4064) (layer "B.Cu") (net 30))
 (segment (start 30.226 58.114762) (end 30.962381 57.378381) (width 0.4064) (layer "B.Cu") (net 30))
 (segment (start 35.226 72.3484) (end 44.4116 81.534) (width 0.4064) (layer "B.Cu") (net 30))
 (segment (start 78.232 43.434) (end 74.8 40.002) (width 0.4064) (layer "B.Cu") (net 30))
 (segment (start 72.898 46.228) (end 71.752 45.082) (width 0.4064) (layer "B.Cu") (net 28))
 (segment (start 73.152 46.228) (end 72.898 46.228) (width 0.4064) (layer "B.Cu") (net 28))
 (segment (start 71.752 45.082) (end 64.331 45.082) (width 0.4064) (layer "B.Cu") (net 28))
 (segment (start 74.168 50.038) (end 74.168 50.292) (width 0.2) (layer "B.Cu") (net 27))
 (segment (start 71.758 50.162) (end 64.331 50.162) (width 0.4064) (layer "B.Cu") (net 27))
 (segment (start 64.455 50.038) (end 64.331 50.162) (width 0.2) (layer "B.Cu") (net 27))
 (segment (start 73.152 48.768) (end 71.758 50.162) (width 0.4064) (layer "B.Cu") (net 27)))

